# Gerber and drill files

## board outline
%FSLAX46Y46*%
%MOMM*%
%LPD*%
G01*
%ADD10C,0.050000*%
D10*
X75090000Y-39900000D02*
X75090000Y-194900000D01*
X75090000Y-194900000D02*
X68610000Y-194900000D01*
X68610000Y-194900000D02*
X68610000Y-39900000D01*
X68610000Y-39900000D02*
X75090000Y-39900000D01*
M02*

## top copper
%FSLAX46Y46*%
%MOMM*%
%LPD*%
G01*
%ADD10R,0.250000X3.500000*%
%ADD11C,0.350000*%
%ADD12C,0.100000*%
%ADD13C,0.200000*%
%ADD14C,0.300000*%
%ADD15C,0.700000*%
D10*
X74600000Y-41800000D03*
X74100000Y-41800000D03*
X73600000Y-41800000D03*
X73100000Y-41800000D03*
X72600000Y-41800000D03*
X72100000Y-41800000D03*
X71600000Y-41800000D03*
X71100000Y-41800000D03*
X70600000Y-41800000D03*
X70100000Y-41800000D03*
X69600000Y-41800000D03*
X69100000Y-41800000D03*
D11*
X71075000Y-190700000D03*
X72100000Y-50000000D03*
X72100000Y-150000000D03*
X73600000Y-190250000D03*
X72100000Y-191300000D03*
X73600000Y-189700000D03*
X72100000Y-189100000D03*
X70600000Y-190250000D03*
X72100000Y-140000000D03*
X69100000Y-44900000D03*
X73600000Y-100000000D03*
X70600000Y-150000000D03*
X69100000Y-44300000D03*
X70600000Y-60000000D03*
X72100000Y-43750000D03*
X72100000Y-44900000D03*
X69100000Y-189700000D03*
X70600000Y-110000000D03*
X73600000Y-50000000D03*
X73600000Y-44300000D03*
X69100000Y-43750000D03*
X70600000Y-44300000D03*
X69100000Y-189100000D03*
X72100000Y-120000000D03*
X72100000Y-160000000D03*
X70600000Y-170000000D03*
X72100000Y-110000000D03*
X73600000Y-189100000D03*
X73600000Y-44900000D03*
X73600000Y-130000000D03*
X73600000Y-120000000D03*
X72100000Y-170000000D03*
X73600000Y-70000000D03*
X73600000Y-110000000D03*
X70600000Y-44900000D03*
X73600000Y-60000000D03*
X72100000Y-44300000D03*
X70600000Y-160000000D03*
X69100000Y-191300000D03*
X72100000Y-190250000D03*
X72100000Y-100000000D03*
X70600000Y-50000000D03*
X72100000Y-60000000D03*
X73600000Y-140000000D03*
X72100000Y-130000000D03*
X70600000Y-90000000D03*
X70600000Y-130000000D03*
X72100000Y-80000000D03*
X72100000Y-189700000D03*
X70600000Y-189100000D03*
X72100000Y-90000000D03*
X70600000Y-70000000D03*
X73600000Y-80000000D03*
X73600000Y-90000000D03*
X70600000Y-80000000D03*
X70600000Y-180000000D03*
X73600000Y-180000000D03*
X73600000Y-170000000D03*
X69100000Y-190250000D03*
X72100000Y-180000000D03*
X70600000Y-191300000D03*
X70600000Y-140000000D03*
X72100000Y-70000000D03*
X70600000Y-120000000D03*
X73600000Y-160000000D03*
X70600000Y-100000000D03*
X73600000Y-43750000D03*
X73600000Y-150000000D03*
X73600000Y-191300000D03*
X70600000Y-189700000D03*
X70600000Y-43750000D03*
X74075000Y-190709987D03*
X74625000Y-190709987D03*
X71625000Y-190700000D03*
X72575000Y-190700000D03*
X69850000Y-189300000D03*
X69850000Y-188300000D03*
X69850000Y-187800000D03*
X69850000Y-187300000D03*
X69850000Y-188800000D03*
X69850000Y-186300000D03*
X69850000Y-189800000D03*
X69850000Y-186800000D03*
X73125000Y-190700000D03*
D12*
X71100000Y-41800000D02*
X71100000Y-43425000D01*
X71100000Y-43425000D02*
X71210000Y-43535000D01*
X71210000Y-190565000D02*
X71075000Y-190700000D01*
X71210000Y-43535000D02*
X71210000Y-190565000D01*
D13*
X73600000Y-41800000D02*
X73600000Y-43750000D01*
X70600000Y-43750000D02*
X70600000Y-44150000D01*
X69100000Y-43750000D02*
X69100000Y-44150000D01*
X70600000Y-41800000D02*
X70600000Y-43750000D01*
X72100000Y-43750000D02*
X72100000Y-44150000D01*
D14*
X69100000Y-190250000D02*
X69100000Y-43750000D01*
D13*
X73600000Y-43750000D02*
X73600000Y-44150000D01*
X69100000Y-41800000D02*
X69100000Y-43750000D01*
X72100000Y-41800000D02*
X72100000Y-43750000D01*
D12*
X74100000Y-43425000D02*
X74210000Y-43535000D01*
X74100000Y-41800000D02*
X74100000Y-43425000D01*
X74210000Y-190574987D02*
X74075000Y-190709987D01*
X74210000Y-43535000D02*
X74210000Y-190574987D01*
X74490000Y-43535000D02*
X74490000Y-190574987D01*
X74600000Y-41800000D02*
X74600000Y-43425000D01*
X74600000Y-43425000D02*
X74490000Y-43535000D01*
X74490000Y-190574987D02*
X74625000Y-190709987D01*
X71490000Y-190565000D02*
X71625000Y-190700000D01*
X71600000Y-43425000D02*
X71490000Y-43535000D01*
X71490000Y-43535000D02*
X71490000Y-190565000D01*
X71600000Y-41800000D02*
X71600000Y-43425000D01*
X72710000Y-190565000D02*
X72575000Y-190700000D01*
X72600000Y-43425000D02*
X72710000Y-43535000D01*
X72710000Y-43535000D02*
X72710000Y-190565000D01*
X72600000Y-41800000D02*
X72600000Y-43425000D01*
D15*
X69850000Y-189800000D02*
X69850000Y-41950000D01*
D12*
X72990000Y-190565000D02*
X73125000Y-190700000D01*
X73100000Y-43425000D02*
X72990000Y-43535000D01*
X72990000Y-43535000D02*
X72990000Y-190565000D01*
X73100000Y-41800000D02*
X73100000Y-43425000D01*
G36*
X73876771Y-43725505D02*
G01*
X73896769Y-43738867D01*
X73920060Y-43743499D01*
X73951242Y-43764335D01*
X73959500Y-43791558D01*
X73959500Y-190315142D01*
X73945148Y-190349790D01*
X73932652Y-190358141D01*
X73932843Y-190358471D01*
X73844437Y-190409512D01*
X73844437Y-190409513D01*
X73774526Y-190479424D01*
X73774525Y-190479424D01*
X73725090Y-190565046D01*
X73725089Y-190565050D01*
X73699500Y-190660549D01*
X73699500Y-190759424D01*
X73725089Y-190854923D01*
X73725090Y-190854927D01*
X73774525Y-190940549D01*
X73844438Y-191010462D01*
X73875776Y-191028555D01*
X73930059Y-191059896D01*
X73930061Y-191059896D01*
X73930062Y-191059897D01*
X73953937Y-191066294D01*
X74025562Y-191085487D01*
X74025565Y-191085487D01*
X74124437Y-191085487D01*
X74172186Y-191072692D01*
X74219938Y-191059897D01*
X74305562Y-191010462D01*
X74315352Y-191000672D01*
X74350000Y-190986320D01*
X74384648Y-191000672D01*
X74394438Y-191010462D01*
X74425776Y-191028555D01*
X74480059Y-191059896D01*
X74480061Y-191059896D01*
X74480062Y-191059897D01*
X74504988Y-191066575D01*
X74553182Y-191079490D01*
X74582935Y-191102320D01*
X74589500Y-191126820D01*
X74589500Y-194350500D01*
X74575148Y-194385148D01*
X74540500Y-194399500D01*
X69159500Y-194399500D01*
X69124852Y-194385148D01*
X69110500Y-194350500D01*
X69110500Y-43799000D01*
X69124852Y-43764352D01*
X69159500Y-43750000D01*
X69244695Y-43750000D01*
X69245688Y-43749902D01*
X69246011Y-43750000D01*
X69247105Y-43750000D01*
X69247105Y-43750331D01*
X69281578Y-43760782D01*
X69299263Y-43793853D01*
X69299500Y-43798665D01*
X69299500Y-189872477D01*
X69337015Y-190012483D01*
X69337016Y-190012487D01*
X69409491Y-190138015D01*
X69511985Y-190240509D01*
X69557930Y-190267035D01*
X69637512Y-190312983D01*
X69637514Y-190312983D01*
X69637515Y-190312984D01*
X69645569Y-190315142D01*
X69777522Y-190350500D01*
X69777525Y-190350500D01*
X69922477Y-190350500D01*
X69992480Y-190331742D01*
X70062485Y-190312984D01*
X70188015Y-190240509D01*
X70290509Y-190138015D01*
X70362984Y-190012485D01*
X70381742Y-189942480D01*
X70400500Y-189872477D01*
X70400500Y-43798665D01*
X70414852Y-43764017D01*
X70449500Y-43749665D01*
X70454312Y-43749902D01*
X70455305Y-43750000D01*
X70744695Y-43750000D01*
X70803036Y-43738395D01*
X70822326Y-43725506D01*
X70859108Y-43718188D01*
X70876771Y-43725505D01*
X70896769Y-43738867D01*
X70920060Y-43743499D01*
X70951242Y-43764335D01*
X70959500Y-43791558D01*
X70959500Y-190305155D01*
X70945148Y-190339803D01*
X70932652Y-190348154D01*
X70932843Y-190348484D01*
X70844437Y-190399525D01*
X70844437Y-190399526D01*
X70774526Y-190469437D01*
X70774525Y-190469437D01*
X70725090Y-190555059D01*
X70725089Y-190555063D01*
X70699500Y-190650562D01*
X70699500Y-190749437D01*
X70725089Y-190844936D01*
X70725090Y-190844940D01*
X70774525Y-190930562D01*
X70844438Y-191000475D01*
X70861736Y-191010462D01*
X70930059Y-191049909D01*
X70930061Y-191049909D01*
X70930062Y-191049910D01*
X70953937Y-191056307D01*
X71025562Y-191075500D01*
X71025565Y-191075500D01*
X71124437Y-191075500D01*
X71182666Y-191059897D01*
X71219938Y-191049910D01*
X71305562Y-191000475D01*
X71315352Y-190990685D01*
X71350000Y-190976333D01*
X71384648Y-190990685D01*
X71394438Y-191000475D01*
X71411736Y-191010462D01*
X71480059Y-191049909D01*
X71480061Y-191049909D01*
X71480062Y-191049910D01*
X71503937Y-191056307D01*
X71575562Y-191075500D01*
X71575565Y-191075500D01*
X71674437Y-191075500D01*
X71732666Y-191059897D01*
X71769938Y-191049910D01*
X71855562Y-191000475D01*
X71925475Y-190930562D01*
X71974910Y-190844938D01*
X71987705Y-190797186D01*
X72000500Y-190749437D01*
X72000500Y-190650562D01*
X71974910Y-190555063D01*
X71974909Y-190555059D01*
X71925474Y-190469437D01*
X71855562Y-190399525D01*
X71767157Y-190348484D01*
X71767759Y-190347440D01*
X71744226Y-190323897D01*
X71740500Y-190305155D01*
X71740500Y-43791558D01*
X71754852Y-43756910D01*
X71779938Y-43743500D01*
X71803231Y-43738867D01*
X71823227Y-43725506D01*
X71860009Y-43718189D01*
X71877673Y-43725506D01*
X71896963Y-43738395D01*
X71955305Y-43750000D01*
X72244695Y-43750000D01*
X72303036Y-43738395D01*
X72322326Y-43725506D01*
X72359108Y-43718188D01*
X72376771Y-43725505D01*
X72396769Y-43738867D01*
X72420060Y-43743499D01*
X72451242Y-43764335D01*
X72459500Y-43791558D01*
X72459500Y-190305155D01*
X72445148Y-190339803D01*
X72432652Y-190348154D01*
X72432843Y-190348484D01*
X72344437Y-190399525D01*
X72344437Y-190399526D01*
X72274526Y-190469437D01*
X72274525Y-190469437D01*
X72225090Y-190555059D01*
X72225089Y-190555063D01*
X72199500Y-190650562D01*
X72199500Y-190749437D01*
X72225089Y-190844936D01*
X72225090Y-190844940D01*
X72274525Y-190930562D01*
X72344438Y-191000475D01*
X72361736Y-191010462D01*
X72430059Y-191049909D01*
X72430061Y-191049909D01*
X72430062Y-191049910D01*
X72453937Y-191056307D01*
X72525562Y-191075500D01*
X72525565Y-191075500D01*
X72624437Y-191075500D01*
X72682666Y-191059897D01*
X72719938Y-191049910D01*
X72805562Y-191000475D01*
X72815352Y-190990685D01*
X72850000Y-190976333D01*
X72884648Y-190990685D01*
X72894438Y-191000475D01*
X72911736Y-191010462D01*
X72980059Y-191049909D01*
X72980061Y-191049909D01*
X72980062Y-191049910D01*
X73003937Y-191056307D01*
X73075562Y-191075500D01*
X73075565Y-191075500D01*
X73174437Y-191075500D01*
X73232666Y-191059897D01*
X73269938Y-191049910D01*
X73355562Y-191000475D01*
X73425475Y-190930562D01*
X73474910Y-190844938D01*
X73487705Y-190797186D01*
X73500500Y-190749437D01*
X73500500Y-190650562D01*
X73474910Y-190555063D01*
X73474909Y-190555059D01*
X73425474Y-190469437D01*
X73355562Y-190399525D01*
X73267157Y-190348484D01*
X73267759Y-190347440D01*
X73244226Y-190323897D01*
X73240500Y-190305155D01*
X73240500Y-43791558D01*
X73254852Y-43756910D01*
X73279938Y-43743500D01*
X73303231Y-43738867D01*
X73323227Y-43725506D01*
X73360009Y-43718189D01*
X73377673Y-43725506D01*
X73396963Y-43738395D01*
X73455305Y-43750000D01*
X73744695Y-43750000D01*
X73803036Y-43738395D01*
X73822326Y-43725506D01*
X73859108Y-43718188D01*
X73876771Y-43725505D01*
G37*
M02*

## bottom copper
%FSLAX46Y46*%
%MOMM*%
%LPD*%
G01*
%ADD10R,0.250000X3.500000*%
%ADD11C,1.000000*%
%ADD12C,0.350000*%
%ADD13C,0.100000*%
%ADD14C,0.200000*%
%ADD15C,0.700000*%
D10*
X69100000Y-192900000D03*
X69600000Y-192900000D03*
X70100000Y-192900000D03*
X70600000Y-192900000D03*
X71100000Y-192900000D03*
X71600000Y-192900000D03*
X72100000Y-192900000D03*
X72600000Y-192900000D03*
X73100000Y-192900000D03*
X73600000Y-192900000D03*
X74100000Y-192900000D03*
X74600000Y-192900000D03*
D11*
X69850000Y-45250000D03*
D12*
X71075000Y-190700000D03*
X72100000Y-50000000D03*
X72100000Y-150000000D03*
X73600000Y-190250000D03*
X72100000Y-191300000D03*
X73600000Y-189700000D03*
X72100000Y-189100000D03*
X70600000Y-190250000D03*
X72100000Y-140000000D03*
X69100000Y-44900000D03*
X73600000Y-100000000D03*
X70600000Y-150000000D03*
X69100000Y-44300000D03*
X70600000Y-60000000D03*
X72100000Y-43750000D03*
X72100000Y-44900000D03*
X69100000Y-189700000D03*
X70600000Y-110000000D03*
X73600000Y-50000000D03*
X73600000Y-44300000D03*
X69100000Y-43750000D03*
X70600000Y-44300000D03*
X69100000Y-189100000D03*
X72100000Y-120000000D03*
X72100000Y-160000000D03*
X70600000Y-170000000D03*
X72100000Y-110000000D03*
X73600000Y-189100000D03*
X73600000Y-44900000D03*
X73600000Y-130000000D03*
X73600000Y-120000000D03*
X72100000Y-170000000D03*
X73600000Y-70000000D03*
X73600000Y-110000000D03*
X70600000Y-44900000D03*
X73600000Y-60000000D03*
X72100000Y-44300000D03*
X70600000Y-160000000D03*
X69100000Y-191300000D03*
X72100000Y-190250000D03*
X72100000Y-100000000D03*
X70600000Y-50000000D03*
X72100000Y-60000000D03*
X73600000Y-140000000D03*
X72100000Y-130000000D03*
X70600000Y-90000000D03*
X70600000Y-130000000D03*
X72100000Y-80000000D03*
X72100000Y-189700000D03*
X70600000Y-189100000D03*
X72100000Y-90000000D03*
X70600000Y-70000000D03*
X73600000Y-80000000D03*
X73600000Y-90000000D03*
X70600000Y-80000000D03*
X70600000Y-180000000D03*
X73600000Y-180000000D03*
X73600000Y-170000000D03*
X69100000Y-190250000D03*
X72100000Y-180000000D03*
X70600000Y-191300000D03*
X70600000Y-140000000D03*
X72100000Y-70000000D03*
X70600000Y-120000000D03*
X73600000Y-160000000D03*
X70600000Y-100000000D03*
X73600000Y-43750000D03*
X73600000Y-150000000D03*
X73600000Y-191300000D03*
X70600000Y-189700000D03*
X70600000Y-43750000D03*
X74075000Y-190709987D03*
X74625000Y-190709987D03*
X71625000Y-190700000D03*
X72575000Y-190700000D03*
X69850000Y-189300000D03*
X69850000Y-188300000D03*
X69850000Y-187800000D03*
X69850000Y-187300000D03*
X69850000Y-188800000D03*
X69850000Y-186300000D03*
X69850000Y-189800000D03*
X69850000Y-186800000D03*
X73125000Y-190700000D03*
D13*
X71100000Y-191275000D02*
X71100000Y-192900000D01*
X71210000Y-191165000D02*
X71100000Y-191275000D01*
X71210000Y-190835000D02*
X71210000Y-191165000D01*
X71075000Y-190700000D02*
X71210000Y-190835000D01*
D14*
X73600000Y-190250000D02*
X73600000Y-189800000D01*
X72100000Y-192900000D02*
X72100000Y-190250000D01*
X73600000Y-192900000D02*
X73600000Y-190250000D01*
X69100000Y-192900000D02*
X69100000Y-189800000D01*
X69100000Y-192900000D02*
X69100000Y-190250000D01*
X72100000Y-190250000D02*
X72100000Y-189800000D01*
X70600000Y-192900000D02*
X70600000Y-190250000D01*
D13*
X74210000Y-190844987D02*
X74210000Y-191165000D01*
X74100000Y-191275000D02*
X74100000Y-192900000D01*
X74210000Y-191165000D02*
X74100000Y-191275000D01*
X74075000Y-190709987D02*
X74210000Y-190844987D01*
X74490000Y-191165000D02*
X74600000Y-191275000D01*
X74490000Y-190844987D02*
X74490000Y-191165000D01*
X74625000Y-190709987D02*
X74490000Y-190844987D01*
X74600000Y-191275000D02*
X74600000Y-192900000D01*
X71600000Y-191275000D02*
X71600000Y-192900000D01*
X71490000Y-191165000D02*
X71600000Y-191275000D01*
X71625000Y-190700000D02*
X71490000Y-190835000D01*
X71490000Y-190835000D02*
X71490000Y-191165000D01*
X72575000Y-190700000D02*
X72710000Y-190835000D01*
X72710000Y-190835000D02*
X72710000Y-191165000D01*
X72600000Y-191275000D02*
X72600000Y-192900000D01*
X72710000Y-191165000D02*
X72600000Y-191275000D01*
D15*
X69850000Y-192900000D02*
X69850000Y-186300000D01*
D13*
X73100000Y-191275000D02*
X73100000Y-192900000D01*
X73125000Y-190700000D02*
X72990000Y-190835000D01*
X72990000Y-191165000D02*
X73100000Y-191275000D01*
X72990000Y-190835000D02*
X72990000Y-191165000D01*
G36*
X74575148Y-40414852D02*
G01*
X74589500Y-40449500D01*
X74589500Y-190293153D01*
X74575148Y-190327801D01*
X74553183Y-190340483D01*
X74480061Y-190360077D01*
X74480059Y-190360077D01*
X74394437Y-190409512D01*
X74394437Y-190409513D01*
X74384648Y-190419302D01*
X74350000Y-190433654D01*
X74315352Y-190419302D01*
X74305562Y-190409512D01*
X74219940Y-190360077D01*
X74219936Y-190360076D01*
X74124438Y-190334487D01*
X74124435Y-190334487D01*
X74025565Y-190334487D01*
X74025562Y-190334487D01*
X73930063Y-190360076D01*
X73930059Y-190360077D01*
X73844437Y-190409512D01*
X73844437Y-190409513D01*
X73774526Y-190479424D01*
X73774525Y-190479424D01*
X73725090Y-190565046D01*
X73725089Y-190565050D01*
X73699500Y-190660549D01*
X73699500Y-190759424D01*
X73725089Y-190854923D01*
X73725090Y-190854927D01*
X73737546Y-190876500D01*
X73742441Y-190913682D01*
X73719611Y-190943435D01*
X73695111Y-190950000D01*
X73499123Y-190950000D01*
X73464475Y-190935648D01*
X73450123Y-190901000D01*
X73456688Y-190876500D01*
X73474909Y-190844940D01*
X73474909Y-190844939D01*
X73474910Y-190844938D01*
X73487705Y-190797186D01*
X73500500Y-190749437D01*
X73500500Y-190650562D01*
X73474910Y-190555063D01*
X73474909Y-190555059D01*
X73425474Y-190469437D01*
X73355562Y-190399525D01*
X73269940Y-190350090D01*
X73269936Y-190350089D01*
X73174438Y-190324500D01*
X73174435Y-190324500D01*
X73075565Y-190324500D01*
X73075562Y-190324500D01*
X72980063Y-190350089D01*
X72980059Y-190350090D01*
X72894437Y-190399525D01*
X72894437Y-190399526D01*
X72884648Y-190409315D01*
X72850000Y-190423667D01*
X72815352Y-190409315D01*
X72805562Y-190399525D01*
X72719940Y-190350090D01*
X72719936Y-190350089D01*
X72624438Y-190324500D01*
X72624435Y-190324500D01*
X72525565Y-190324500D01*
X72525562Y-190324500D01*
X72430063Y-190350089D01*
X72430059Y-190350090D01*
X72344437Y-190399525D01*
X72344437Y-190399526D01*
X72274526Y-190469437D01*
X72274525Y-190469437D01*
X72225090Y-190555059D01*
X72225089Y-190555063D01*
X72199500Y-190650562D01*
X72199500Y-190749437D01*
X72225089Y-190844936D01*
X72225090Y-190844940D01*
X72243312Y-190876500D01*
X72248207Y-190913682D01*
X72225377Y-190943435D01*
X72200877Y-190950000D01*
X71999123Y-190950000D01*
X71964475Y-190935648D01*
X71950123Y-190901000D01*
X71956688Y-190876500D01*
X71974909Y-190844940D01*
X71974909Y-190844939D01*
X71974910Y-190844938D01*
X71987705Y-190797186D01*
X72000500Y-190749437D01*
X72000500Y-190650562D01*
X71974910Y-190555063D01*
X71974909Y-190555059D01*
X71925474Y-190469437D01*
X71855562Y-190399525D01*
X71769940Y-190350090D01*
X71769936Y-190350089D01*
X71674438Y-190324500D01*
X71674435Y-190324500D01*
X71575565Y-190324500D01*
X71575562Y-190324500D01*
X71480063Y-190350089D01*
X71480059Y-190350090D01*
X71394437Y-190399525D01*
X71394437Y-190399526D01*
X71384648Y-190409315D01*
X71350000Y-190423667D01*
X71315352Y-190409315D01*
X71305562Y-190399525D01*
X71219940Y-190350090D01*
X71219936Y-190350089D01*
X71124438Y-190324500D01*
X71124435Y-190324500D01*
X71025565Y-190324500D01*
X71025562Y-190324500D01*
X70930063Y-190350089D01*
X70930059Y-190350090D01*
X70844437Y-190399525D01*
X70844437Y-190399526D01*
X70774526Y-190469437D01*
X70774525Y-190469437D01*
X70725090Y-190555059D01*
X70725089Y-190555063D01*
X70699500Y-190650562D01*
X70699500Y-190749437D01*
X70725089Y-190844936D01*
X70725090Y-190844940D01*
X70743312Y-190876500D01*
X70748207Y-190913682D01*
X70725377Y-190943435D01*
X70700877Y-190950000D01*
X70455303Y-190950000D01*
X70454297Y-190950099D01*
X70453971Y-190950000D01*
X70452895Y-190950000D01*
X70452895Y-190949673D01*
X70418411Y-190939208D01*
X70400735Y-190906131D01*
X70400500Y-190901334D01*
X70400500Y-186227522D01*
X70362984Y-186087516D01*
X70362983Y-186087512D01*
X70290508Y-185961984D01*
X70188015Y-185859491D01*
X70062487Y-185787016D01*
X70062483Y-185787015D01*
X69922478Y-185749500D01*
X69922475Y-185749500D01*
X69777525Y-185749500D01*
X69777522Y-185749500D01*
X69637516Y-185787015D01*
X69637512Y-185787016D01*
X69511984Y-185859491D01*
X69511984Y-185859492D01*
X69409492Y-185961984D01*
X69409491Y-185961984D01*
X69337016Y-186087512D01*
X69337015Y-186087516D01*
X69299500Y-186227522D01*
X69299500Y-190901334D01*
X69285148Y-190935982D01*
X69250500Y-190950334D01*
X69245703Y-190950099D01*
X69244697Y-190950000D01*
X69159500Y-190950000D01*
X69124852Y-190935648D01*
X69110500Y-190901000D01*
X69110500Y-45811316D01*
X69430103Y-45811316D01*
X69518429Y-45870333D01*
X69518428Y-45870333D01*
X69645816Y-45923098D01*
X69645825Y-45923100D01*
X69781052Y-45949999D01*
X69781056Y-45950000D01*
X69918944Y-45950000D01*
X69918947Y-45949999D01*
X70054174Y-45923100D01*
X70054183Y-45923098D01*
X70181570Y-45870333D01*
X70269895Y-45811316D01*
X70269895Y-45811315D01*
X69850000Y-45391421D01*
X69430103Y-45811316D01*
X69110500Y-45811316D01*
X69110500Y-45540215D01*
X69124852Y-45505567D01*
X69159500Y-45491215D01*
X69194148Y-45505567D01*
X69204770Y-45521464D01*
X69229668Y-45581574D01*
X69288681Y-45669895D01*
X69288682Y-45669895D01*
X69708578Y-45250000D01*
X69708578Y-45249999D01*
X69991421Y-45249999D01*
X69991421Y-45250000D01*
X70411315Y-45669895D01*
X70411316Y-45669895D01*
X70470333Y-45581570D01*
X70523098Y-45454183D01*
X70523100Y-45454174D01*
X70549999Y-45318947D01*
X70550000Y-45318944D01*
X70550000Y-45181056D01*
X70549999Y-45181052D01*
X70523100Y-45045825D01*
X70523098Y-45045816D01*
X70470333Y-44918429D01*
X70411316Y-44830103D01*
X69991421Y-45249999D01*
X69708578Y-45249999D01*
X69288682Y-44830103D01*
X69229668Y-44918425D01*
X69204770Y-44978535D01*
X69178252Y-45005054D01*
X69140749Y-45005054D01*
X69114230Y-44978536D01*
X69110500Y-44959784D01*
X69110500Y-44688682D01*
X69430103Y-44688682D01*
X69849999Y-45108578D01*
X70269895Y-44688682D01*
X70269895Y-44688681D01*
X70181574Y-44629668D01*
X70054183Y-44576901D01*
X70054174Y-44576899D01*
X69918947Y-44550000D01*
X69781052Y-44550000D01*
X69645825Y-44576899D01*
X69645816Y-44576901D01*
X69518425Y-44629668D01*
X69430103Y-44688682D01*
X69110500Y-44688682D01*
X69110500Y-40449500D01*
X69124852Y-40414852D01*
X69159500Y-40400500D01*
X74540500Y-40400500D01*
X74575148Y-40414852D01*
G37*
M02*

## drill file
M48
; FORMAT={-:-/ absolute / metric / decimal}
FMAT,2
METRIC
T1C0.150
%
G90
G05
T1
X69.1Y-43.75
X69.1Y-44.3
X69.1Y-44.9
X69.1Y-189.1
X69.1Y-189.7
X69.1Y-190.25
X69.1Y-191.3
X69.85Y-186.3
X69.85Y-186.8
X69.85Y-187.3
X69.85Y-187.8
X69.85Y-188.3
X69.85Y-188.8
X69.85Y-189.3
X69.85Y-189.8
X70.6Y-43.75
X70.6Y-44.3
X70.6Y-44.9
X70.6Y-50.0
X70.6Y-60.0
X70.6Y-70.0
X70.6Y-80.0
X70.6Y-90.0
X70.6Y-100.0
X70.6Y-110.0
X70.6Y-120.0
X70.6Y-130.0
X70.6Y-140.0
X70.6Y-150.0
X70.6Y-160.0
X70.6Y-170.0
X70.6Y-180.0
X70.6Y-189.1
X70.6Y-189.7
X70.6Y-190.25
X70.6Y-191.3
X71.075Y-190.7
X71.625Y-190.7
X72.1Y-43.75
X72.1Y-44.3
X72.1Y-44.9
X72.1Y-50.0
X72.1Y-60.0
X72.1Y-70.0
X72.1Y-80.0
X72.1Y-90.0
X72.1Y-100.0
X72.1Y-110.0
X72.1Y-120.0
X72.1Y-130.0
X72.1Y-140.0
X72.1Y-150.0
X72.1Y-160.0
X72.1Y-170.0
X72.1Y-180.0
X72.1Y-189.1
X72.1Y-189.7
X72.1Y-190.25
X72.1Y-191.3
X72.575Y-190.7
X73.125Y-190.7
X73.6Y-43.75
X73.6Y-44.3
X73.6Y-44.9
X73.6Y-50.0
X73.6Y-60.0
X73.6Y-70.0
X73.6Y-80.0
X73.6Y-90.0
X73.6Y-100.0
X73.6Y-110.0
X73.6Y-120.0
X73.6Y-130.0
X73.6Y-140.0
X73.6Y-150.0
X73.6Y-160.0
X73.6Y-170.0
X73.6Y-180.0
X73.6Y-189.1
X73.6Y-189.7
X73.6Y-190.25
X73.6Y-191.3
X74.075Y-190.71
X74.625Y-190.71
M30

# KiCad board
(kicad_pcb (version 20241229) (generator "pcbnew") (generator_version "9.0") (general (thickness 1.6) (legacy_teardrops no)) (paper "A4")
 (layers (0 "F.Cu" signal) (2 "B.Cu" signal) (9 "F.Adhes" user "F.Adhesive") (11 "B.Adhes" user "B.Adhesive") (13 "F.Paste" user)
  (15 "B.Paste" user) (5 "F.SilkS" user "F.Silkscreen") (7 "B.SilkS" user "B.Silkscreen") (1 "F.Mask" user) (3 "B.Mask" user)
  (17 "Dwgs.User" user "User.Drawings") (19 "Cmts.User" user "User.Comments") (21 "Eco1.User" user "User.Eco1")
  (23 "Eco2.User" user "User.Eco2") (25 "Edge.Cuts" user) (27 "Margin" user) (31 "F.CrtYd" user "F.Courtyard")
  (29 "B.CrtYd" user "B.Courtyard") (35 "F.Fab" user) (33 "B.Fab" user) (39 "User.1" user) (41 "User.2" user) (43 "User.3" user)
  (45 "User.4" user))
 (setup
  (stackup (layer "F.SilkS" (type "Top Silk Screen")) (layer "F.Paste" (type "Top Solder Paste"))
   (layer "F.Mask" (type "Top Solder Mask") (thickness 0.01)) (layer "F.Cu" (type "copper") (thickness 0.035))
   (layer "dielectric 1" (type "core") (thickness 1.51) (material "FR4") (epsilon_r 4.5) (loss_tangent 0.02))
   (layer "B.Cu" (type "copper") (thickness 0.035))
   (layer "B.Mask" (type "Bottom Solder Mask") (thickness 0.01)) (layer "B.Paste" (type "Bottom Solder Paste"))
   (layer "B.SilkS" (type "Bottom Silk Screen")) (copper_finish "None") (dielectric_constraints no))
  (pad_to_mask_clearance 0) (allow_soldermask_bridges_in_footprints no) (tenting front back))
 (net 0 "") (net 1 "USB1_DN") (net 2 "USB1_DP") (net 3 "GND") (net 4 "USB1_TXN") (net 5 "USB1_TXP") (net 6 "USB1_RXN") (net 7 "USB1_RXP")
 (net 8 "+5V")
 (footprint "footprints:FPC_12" (layer "F.Cu") (at 71.85 41.8)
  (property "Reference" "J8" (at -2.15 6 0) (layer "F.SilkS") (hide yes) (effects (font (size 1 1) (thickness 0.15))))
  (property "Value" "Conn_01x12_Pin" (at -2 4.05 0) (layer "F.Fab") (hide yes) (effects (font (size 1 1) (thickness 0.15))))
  (pad "1" smd rect (at 2.75 0) (size 0.25 3.5) (layers "F.Cu" "F.Mask" "F.Paste") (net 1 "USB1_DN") (thermal_bridge_angle 45))
  (pad "2" smd rect (at 2.25 0) (size 0.25 3.5) (layers "F.Cu" "F.Mask" "F.Paste") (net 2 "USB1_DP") (thermal_bridge_angle 45))
  (pad "3" smd rect (at 1.75 0) (size 0.25 3.5) (layers "F.Cu" "F.Mask" "F.Paste") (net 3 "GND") (thermal_bridge_angle 45))
  (pad "4" smd rect (at 1.25 0) (size 0.25 3.5) (layers "F.Cu" "F.Mask" "F.Paste") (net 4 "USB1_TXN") (thermal_bridge_angle 45))
  (pad "5" smd rect (at 0.75 0) (size 0.25 3.5) (layers "F.Cu" "F.Mask" "F.Paste") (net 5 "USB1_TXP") (thermal_bridge_angle 45))
  (pad "6" smd rect (at 0.25 0) (size 0.25 3.5) (layers "F.Cu" "F.Mask" "F.Paste") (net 3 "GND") (thermal_bridge_angle 45))
  (pad "7" smd rect (at -0.25 0) (size 0.25 3.5) (layers "F.Cu" "F.Mask" "F.Paste") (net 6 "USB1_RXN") (thermal_bridge_angle 45))
  (pad "8" smd rect (at -0.75 0) (size 0.25 3.5) (layers "F.Cu" "F.Mask" "F.Paste") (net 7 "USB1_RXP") (thermal_bridge_angle 45))
  (pad "9" smd rect (at -1.25 0) (size 0.25 3.5) (layers "F.Cu" "F.Mask" "F.Paste") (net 3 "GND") (thermal_bridge_angle 45))
  (pad "10" smd rect (at -1.75 0) (size 0.25 3.5) (layers "F.Cu" "F.Mask" "F.Paste") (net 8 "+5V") (thermal_bridge_angle 45))
  (pad "11" smd rect (at -2.25 0) (size 0.25 3.5) (layers "F.Cu" "F.Mask" "F.Paste") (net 8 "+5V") (thermal_bridge_angle 45))
  (pad "12" smd rect (at -2.75 0) (size 0.25 3.5) (layers "F.Cu" "F.Mask" "F.Paste") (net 3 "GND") (thermal_bridge_angle 45)))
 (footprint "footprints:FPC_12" (layer "B.Cu") (at 71.85 192.9 180)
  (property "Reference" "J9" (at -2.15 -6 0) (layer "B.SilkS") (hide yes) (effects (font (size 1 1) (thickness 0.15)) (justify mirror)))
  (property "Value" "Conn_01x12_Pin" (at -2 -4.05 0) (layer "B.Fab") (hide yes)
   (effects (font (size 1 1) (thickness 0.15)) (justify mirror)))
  (pad "1" smd rect (at 2.75 0 180) (size 0.25 3.5) (layers "B.Cu" "B.Mask" "B.Paste") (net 3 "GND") (thermal_bridge_angle 45))
  (pad "2" smd rect (at 2.25 0 180) (size 0.25 3.5) (layers "B.Cu" "B.Mask" "B.Paste") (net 8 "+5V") (thermal_bridge_angle 45))
  (pad "3" smd rect (at 1.75 0 180) (size 0.25 3.5) (layers "B.Cu" "B.Mask" "B.Paste") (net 8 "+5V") (thermal_bridge_angle 45))
  (pad "4" smd rect (at 1.25 0 180) (size 0.25 3.5) (layers "B.Cu" "B.Mask" "B.Paste") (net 3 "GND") (thermal_bridge_angle 45))
  (pad "5" smd rect (at 0.75 0 180) (size 0.25 3.5) (layers "B.Cu" "B.Mask" "B.Paste") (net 7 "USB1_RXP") (thermal_bridge_angle 45))
  (pad "6" smd rect (at 0.25 0 180) (size 0.25 3.5) (layers "B.Cu" "B.Mask" "B.Paste") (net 6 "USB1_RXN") (thermal_bridge_angle 45))
  (pad "7" smd rect (at -0.25 0 180) (size 0.25 3.5) (layers "B.Cu" "B.Mask" "B.Paste") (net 3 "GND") (thermal_bridge_angle 45))
  (pad "8" smd rect (at -0.75 0 180) (size 0.25 3.5) (layers "B.Cu" "B.Mask" "B.Paste") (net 5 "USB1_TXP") (thermal_bridge_angle 45))
  (pad "9" smd rect (at -1.25 0 180) (size 0.25 3.5) (layers "B.Cu" "B.Mask" "B.Paste") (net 4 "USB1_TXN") (thermal_bridge_angle 45))
  (pad "10" smd rect (at -1.75 0 180) (size 0.25 3.5) (layers "B.Cu" "B.Mask" "B.Paste") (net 3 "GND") (thermal_bridge_angle 45))
  (pad "11" smd rect (at -2.25 0 180) (size 0.25 3.5) (layers "B.Cu" "B.Mask" "B.Paste") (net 2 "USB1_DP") (thermal_bridge_angle 45))
  (pad "12" smd rect (at -2.75 0 180) (size 0.25 3.5) (layers "B.Cu" "B.Mask" "B.Paste") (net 1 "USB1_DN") (thermal_bridge_angle 45)))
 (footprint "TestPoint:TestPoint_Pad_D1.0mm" (layer "B.Cu") (at 69.85 45.25 180)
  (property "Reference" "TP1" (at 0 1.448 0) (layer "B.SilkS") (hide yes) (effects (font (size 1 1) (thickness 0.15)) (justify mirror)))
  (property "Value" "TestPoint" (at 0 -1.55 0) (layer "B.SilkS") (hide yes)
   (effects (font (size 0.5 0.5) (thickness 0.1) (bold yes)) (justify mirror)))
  (pad "1" smd circle (at 0 0 180) (size 1 1) (layers "B.Cu" "B.Mask") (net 3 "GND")))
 (gr_line (start 75.09 39.9) (end 75.09 194.9) (stroke (width 0.05) (type solid)) (layer "Edge.Cuts"))
 (gr_line (start 75.09 194.9) (end 68.61 194.9) (stroke (width 0.05) (type solid)) (layer "Edge.Cuts"))
 (gr_line (start 68.61 194.9) (end 68.61 39.9) (stroke (width 0.05) (type solid)) (layer "Edge.Cuts"))
 (gr_line (start 68.61 39.9) (end 75.09 39.9) (stroke (width 0.05) (type solid)) (layer "Edge.Cuts"))
 (segment (start 71.1 41.8) (end 71.1 43.425) (width 0.1) (layer "F.Cu") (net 7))
 (segment (start 71.1 43.425) (end 71.21 43.535) (width 0.1) (layer "F.Cu") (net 7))
 (segment (start 71.21 190.565) (end 71.075 190.7) (width 0.1) (layer "F.Cu") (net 7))
 (segment (start 71.21 43.535) (end 71.21 190.565) (width 0.1) (layer "F.Cu") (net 7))
 (via (at 71.075 190.7) (size 0.35) (drill 0.15) (layers "F.Cu" "B.Cu") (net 7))
 (segment (start 71.1 191.275) (end 71.1 192.9) (width 0.1) (layer "B.Cu") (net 7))
 (segment (start 71.21 191.165) (end 71.1 191.275) (width 0.1) (layer "B.Cu") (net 7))
 (segment (start 71.21 190.835) (end 71.21 191.165) (width 0.1) (layer "B.Cu") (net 7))
 (segment (start 71.075 190.7) (end 71.21 190.835) (width 0.1) (layer "B.Cu") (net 7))
 (segment (start 73.6 41.8) (end 73.6 43.75) (width 0.2) (layer "F.Cu") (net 3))
 (segment (start 70.6 43.75) (end 70.6 44.15) (width 0.2) (layer "F.Cu") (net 3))
 (segment (start 69.1 43.75) (end 69.1 44.15) (width 0.2) (layer "F.Cu") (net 3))
 (segment (start 70.6 41.8) (end 70.6 43.75) (width 0.2) (layer "F.Cu") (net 3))
 (segment (start 72.1 43.75) (end 72.1 44.15) (width 0.2) (layer "F.Cu") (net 3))
 (segment (start 69.1 190.25) (end 69.1 43.75) (width 0.3) (layer "F.Cu") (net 3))
 (segment (start 73.6 43.75) (end 73.6 44.15) (width 0.2) (layer "F.Cu") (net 3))
 (segment (start 69.1 41.8) (end 69.1 43.75) (width 0.2) (layer "F.Cu") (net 3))
 (segment (start 72.1 41.8) (end 72.1 43.75) (width 0.2) (layer "F.Cu") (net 3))
 (via (at 72.1 50) (size 0.35) (drill 0.15) (layers "F.Cu" "B.Cu") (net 3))
 (via (at 72.1 150) (size 0.35) (drill 0.15) (layers "F.Cu" "B.Cu") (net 3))
 (via (at 73.6 190.25) (size 0.35) (drill 0.15) (layers "F.Cu" "B.Cu") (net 3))
 (via (at 72.1 191.3) (size 0.35) (drill 0.15) (layers "F.Cu" "B.Cu") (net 3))
 (via (at 73.6 189.7) (size 0.35) (drill 0.15) (layers "F.Cu" "B.Cu") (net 3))
 (via (at 72.1 189.1) (size 0.35) (drill 0.15) (layers "F.Cu" "B.Cu") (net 3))
 (via (at 70.6 190.25) (size 0.35) (drill 0.15) (layers "F.Cu" "B.Cu") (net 3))
 (via (at 72.1 140) (size 0.35) (drill 0.15) (layers "F.Cu" "B.Cu") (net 3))
 (via (at 69.1 44.9) (size 0.35) (drill 0.15) (layers "F.Cu" "B.Cu") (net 3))
 (via (at 73.6 100) (size 0.35) (drill 0.15) (layers "F.Cu" "B.Cu") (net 3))
 (via (at 70.6 150) (size 0.35) (drill 0.15) (layers "F.Cu" "B.Cu") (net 3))
 (via (at 69.1 44.3) (size 0.35) (drill 0.15) (layers "F.Cu" "B.Cu") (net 3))
 (via (at 70.6 60) (size 0.35) (drill 0.15) (layers "F.Cu" "B.Cu") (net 3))
 (via (at 72.1 43.75) (size 0.35) (drill 0.15) (layers "F.Cu" "B.Cu") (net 3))
 (via (at 72.1 44.9) (size 0.35) (drill 0.15) (layers "F.Cu" "B.Cu") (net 3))
 (via (at 69.1 189.7) (size 0.35) (drill 0.15) (layers "F.Cu" "B.Cu") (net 3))
 (via (at 70.6 110) (size 0.35) (drill 0.15) (layers "F.Cu" "B.Cu") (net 3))
 (via (at 73.6 50) (size 0.35) (drill 0.15) (layers "F.Cu" "B.Cu") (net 3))
 (via (at 73.6 44.3) (size 0.35) (drill 0.15) (layers "F.Cu" "B.Cu") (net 3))
 (via (at 69.1 43.75) (size 0.35) (drill 0.15) (layers "F.Cu" "B.Cu") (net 3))
 (via (at 70.6 44.3) (size 0.35) (drill 0.15) (layers "F.Cu" "B.Cu") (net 3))
 (via (at 69.1 189.1) (size 0.35) (drill 0.15) (layers "F.Cu" "B.Cu") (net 3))
 (via (at 72.1 120) (size 0.35) (drill 0.15) (layers "F.Cu" "B.Cu") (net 3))
 (via (at 72.1 160) (size 0.35) (drill 0.15) (layers "F.Cu" "B.Cu") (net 3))
 (via (at 70.6 170) (size 0.35) (drill 0.15) (layers "F.Cu" "B.Cu") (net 3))
 (via (at 72.1 110) (size 0.35) (drill 0.15) (layers "F.Cu" "B.Cu") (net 3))
 (via (at 73.6 189.1) (size 0.35) (drill 0.15) (layers "F.Cu" "B.Cu") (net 3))
 (via (at 73.6 44.9) (size 0.35) (drill 0.15) (layers "F.Cu" "B.Cu") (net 3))
 (via (at 73.6 130) (size 0.35) (drill 0.15) (layers "F.Cu" "B.Cu") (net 3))
 (via (at 73.6 120) (size 0.35) (drill 0.15) (layers "F.Cu" "B.Cu") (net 3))
 (via (at 72.1 170) (size 0.35) (drill 0.15) (layers "F.Cu" "B.Cu") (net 3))
 (via (at 73.6 70) (size 0.35) (drill 0.15) (layers "F.Cu" "B.Cu") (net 3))
 (via (at 73.6 110) (size 0.35) (drill 0.15) (layers "F.Cu" "B.Cu") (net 3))
 (via (at 70.6 44.9) (size 0.35) (drill 0.15) (layers "F.Cu" "B.Cu") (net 3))
 (via (at 73.6 60) (size 0.35) (drill 0.15) (layers "F.Cu" "B.Cu") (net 3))
 (via (at 72.1 44.3) (size 0.35) (drill 0.15) (layers "F.Cu" "B.Cu") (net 3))
 (via (at 70.6 160) (size 0.35) (drill 0.15) (layers "F.Cu" "B.Cu") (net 3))
 (via (at 69.1 191.3) (size 0.35) (drill 0.15) (layers "F.Cu" "B.Cu") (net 3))
 (via (at 72.1 190.25) (size 0.35) (drill 0.15) (layers "F.Cu" "B.Cu") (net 3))
 (via (at 72.1 100) (size 0.35) (drill 0.15) (layers "F.Cu" "B.Cu") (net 3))
 (via (at 70.6 50) (size 0.35) (drill 0.15) (layers "F.Cu" "B.Cu") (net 3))
 (via (at 72.1 60) (size 0.35) (drill 0.15) (layers "F.Cu" "B.Cu") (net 3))
 (via (at 73.6 140) (size 0.35) (drill 0.15) (layers "F.Cu" "B.Cu") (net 3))
 (via (at 72.1 130) (size 0.35) (drill 0.15) (layers "F.Cu" "B.Cu") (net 3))
 (via (at 70.6 90) (size 0.35) (drill 0.15) (layers "F.Cu" "B.Cu") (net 3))
 (via (at 70.6 130) (size 0.35) (drill 0.15) (layers "F.Cu" "B.Cu") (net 3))
 (via (at 72.1 80) (size 0.35) (drill 0.15) (layers "F.Cu" "B.Cu") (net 3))
 (via (at 72.1 189.7) (size 0.35) (drill 0.15) (layers "F.Cu" "B.Cu") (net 3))
 (via (at 70.6 189.1) (size 0.35) (drill 0.15) (layers "F.Cu" "B.Cu") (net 3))
 (via (at 72.1 90) (size 0.35) (drill 0.15) (layers "F.Cu" "B.Cu") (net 3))
 (via (at 70.6 70) (size 0.35) (drill 0.15) (layers "F.Cu" "B.Cu") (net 3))
 (via (at 73.6 80) (size 0.35) (drill 0.15) (layers "F.Cu" "B.Cu") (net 3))
 (via (at 73.6 90) (size 0.35) (drill 0.15) (layers "F.Cu" "B.Cu") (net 3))
 (via (at 70.6 80) (size 0.35) (drill 0.15) (layers "F.Cu" "B.Cu") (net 3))
 (via (at 70.6 180) (size 0.35) (drill 0.15) (layers "F.Cu" "B.Cu") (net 3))
 (via (at 73.6 180) (size 0.35) (drill 0.15) (layers "F.Cu" "B.Cu") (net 3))
 (via (at 73.6 170) (size 0.35) (drill 0.15) (layers "F.Cu" "B.Cu") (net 3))
 (via (at 69.1 190.25) (size 0.35) (drill 0.15) (layers "F.Cu" "B.Cu") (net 3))
 (via (at 72.1 180) (size 0.35) (drill 0.15) (layers "F.Cu" "B.Cu") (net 3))
 (via (at 70.6 191.3) (size 0.35) (drill 0.15) (layers "F.Cu" "B.Cu") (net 3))
 (via (at 70.6 140) (size 0.35) (drill 0.15) (layers "F.Cu" "B.Cu") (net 3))
 (via (at 72.1 70) (size 0.35) (drill 0.15) (layers "F.Cu" "B.Cu") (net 3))
 (via (at 70.6 120) (size 0.35) (drill 0.15) (layers "F.Cu" "B.Cu") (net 3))
 (via (at 73.6 160) (size 0.35) (drill 0.15) (layers "F.Cu" "B.Cu") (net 3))
 (via (at 70.6 100) (size 0.35) (drill 0.15) (layers "F.Cu" "B.Cu") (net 3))
 (via (at 73.6 43.75) (size 0.35) (drill 0.15) (layers "F.Cu" "B.Cu") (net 3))
 (via (at 73.6 150) (size 0.35) (drill 0.15) (layers "F.Cu" "B.Cu") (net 3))
 (via (at 73.6 191.3) (size 0.35) (drill 0.15) (layers "F.Cu" "B.Cu") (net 3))
 (via (at 70.6 189.7) (size 0.35) (drill 0.15) (layers "F.Cu" "B.Cu") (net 3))
 (via (at 70.6 43.75) (size 0.35) (drill 0.15) (layers "F.Cu" "B.Cu") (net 3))
 (segment (start 73.6 190.25) (end 73.6 189.8) (width 0.2) (layer "B.Cu") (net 3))
 (segment (start 72.1 192.9) (end 72.1 190.25) (width 0.2) (layer "B.Cu") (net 3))
 (segment (start 73.6 192.9) (end 73.6 190.25) (width 0.2) (layer "B.Cu") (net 3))
 (segment (start 69.1 192.9) (end 69.1 189.8) (width 0.2) (layer "B.Cu") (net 3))
 (segment (start 69.1 192.9) (end 69.1 190.25) (width 0.2) (layer "B.Cu") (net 3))
 (segment (start 72.1 190.25) (end 72.1 189.8) (width 0.2) (layer "B.Cu") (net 3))
 (segment (start 70.6 192.9) (end 70.6 190.25) (width 0.2) (layer "B.Cu") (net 3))
 (segment (start 74.1 43.425) (end 74.21 43.535) (width 0.1) (layer "F.Cu") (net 2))
 (segment (start 74.1 41.8) (end 74.1 43.425) (width 0.1) (layer "F.Cu") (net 2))
 (segment (start 74.21 190.574987) (end 74.075 190.709987) (width 0.1) (layer "F.Cu") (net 2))
 (segment (start 74.21 43.535) (end 74.21 190.574987) (width 0.1) (layer "F.Cu") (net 2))
 (via (at 74.075 190.709987) (size 0.35) (drill 0.15) (layers "F.Cu" "B.Cu") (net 2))
 (segment (start 74.21 190.844987) (end 74.21 191.165) (width 0.1) (layer "B.Cu") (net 2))
 (segment (start 74.1 191.275) (end 74.1 192.9) (width 0.1) (layer "B.Cu") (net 2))
 (segment (start 74.21 191.165) (end 74.1 191.275) (width 0.1) (layer "B.Cu") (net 2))
 (segment (start 74.075 190.709987) (end 74.21 190.844987) (width 0.1) (layer "B.Cu") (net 2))
 (segment (start 74.49 43.535) (end 74.49 190.574987) (width 0.1) (layer "F.Cu") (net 1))
 (segment (start 74.6 41.8) (end 74.6 43.425) (width 0.1) (layer "F.Cu") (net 1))
 (segment (start 74.6 43.425) (end 74.49 43.535) (width 0.1) (layer "F.Cu") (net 1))
 (segment (start 74.49 190.574987) (end 74.625 190.709987) (width 0.1) (layer "F.Cu") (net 1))
 (via (at 74.625 190.709987) (size 0.35) (drill 0.15) (layers "F.Cu" "B.Cu") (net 1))
 (segment (start 74.49 191.165) (end 74.6 191.275) (width 0.1) (layer "B.Cu") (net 1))
 (segment (start 74.49 190.844987) (end 74.49 191.165) (width 0.1) (layer "B.Cu") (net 1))
 (segment (start 74.625 190.709987) (end 74.49 190.844987) (width 0.1) (layer "B.Cu") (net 1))
 (segment (start 74.6 191.275) (end 74.6 192.9) (width 0.1) (layer "B.Cu") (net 1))
 (segment (start 71.49 190.565) (end 71.625 190.7) (width 0.1) (layer "F.Cu") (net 6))
 (segment (start 71.6 43.425) (end 71.49 43.535) (width 0.1) (layer "F.Cu") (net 6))
 (segment (start 71.49 43.535) (end 71.49 190.565) (width 0.1) (layer "F.Cu") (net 6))
 (segment (start 71.6 41.8) (end 71.6 43.425) (width 0.1) (layer "F.Cu") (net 6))
 (via (at 71.625 190.7) (size 0.35) (drill 0.15) (layers "F.Cu" "B.Cu") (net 6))
 (segment (start 71.6 191.275) (end 71.6 192.9) (width 0.1) (layer "B.Cu") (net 6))
 (segment (start 71.49 191.165) (end 71.6 191.275) (width 0.1) (layer "B.Cu") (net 6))
 (segment (start 71.625 190.7) (end 71.49 190.835) (width 0.1) (layer "B.Cu") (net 6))
 (segment (start 71.49 190.835) (end 71.49 191.165) (width 0.1) (layer "B.Cu") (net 6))
 (segment (start 72.71 190.565) (end 72.575 190.7) (width 0.1) (layer "F.Cu") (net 5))
 (segment (start 72.6 43.425) (end 72.71 43.535) (width 0.1) (layer "F.Cu") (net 5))
 (segment (start 72.71 43.535) (end 72.71 190.565) (width 0.1) (layer "F.Cu") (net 5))
 (segment (start 72.6 41.8) (end 72.6 43.425) (width 0.1) (layer "F.Cu") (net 5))
 (via (at 72.575 190.7) (size 0.35) (drill 0.15) (layers "F.Cu" "B.Cu") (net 5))
 (segment (start 72.575 190.7) (end 72.71 190.835) (width 0.1) (layer "B.Cu") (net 5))
 (segment (start 72.71 190.835) (end 72.71 191.165) (width 0.1) (layer "B.Cu") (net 5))
 (segment (start 72.6 191.275) (end 72.6 192.9) (width 0.1) (layer "B.Cu") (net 5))
 (segment (start 72.71 191.165) (end 72.6 191.275) (width 0.1) (layer "B.Cu") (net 5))
 (segment (start 69.85 189.8) (end 69.85 41.95) (width 0.7) (layer "F.Cu") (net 8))
 (via (at 69.85 189.3) (size 0.35) (drill 0.15) (layers "F.Cu" "B.Cu") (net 8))
 (via (at 69.85 188.3) (size 0.35) (drill 0.15) (layers "F.Cu" "B.Cu") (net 8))
 (via (at 69.85 187.8) (size 0.35) (drill 0.15) (layers "F.Cu" "B.Cu") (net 8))
 (via (at 69.85 187.3) (size 0.35) (drill 0.15) (layers "F.Cu" "B.Cu") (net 8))
 (via (at 69.85 188.8) (size 0.35) (drill 0.15) (layers "F.Cu" "B.Cu") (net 8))
 (via (at 69.85 186.3) (size 0.35) (drill 0.15) (layers "F.Cu" "B.Cu") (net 8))
 (via (at 69.85 189.8) (size 0.35) (drill 0.15) (layers "F.Cu" "B.Cu") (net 8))
 (via (at 69.85 186.8) (size 0.35) (drill 0.15) (layers "F.Cu" "B.Cu") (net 8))
 (segment (start 69.85 192.9) (end 69.85 186.3) (width 0.7) (layer "B.Cu") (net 8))
 (segment (start 72.99 190.565) (end 73.125 190.7) (width 0.1) (layer "F.Cu") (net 4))
 (segment (start 73.1 43.425) (end 72.99 43.535) (width 0.1) (layer "F.Cu") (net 4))
 (segment (start 72.99 43.535) (end 72.99 190.565) (width 0.1) (layer "F.Cu") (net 4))
 (segment (start 73.1 41.8) (end 73.1 43.425) (width 0.1) (layer "F.Cu") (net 4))
 (via (at 73.125 190.7) (size 0.35) (drill 0.15) (layers "F.Cu" "B.Cu") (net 4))
 (segment (start 73.1 191.275) (end 73.1 192.9) (width 0.1) (layer "B.Cu") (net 4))
 (segment (start 73.125 190.7) (end 72.99 190.835) (width 0.1) (layer "B.Cu") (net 4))
 (segment (start 72.99 191.165) (end 73.1 191.275) (width 0.1) (layer "B.Cu") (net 4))
 (segment (start 72.99 190.835) (end 72.99 191.165) (width 0.1) (layer "B.Cu") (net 4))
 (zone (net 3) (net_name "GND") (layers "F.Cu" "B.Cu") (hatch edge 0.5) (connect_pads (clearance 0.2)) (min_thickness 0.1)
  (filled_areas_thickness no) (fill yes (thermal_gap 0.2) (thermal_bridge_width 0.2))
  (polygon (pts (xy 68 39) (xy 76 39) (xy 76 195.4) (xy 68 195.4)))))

